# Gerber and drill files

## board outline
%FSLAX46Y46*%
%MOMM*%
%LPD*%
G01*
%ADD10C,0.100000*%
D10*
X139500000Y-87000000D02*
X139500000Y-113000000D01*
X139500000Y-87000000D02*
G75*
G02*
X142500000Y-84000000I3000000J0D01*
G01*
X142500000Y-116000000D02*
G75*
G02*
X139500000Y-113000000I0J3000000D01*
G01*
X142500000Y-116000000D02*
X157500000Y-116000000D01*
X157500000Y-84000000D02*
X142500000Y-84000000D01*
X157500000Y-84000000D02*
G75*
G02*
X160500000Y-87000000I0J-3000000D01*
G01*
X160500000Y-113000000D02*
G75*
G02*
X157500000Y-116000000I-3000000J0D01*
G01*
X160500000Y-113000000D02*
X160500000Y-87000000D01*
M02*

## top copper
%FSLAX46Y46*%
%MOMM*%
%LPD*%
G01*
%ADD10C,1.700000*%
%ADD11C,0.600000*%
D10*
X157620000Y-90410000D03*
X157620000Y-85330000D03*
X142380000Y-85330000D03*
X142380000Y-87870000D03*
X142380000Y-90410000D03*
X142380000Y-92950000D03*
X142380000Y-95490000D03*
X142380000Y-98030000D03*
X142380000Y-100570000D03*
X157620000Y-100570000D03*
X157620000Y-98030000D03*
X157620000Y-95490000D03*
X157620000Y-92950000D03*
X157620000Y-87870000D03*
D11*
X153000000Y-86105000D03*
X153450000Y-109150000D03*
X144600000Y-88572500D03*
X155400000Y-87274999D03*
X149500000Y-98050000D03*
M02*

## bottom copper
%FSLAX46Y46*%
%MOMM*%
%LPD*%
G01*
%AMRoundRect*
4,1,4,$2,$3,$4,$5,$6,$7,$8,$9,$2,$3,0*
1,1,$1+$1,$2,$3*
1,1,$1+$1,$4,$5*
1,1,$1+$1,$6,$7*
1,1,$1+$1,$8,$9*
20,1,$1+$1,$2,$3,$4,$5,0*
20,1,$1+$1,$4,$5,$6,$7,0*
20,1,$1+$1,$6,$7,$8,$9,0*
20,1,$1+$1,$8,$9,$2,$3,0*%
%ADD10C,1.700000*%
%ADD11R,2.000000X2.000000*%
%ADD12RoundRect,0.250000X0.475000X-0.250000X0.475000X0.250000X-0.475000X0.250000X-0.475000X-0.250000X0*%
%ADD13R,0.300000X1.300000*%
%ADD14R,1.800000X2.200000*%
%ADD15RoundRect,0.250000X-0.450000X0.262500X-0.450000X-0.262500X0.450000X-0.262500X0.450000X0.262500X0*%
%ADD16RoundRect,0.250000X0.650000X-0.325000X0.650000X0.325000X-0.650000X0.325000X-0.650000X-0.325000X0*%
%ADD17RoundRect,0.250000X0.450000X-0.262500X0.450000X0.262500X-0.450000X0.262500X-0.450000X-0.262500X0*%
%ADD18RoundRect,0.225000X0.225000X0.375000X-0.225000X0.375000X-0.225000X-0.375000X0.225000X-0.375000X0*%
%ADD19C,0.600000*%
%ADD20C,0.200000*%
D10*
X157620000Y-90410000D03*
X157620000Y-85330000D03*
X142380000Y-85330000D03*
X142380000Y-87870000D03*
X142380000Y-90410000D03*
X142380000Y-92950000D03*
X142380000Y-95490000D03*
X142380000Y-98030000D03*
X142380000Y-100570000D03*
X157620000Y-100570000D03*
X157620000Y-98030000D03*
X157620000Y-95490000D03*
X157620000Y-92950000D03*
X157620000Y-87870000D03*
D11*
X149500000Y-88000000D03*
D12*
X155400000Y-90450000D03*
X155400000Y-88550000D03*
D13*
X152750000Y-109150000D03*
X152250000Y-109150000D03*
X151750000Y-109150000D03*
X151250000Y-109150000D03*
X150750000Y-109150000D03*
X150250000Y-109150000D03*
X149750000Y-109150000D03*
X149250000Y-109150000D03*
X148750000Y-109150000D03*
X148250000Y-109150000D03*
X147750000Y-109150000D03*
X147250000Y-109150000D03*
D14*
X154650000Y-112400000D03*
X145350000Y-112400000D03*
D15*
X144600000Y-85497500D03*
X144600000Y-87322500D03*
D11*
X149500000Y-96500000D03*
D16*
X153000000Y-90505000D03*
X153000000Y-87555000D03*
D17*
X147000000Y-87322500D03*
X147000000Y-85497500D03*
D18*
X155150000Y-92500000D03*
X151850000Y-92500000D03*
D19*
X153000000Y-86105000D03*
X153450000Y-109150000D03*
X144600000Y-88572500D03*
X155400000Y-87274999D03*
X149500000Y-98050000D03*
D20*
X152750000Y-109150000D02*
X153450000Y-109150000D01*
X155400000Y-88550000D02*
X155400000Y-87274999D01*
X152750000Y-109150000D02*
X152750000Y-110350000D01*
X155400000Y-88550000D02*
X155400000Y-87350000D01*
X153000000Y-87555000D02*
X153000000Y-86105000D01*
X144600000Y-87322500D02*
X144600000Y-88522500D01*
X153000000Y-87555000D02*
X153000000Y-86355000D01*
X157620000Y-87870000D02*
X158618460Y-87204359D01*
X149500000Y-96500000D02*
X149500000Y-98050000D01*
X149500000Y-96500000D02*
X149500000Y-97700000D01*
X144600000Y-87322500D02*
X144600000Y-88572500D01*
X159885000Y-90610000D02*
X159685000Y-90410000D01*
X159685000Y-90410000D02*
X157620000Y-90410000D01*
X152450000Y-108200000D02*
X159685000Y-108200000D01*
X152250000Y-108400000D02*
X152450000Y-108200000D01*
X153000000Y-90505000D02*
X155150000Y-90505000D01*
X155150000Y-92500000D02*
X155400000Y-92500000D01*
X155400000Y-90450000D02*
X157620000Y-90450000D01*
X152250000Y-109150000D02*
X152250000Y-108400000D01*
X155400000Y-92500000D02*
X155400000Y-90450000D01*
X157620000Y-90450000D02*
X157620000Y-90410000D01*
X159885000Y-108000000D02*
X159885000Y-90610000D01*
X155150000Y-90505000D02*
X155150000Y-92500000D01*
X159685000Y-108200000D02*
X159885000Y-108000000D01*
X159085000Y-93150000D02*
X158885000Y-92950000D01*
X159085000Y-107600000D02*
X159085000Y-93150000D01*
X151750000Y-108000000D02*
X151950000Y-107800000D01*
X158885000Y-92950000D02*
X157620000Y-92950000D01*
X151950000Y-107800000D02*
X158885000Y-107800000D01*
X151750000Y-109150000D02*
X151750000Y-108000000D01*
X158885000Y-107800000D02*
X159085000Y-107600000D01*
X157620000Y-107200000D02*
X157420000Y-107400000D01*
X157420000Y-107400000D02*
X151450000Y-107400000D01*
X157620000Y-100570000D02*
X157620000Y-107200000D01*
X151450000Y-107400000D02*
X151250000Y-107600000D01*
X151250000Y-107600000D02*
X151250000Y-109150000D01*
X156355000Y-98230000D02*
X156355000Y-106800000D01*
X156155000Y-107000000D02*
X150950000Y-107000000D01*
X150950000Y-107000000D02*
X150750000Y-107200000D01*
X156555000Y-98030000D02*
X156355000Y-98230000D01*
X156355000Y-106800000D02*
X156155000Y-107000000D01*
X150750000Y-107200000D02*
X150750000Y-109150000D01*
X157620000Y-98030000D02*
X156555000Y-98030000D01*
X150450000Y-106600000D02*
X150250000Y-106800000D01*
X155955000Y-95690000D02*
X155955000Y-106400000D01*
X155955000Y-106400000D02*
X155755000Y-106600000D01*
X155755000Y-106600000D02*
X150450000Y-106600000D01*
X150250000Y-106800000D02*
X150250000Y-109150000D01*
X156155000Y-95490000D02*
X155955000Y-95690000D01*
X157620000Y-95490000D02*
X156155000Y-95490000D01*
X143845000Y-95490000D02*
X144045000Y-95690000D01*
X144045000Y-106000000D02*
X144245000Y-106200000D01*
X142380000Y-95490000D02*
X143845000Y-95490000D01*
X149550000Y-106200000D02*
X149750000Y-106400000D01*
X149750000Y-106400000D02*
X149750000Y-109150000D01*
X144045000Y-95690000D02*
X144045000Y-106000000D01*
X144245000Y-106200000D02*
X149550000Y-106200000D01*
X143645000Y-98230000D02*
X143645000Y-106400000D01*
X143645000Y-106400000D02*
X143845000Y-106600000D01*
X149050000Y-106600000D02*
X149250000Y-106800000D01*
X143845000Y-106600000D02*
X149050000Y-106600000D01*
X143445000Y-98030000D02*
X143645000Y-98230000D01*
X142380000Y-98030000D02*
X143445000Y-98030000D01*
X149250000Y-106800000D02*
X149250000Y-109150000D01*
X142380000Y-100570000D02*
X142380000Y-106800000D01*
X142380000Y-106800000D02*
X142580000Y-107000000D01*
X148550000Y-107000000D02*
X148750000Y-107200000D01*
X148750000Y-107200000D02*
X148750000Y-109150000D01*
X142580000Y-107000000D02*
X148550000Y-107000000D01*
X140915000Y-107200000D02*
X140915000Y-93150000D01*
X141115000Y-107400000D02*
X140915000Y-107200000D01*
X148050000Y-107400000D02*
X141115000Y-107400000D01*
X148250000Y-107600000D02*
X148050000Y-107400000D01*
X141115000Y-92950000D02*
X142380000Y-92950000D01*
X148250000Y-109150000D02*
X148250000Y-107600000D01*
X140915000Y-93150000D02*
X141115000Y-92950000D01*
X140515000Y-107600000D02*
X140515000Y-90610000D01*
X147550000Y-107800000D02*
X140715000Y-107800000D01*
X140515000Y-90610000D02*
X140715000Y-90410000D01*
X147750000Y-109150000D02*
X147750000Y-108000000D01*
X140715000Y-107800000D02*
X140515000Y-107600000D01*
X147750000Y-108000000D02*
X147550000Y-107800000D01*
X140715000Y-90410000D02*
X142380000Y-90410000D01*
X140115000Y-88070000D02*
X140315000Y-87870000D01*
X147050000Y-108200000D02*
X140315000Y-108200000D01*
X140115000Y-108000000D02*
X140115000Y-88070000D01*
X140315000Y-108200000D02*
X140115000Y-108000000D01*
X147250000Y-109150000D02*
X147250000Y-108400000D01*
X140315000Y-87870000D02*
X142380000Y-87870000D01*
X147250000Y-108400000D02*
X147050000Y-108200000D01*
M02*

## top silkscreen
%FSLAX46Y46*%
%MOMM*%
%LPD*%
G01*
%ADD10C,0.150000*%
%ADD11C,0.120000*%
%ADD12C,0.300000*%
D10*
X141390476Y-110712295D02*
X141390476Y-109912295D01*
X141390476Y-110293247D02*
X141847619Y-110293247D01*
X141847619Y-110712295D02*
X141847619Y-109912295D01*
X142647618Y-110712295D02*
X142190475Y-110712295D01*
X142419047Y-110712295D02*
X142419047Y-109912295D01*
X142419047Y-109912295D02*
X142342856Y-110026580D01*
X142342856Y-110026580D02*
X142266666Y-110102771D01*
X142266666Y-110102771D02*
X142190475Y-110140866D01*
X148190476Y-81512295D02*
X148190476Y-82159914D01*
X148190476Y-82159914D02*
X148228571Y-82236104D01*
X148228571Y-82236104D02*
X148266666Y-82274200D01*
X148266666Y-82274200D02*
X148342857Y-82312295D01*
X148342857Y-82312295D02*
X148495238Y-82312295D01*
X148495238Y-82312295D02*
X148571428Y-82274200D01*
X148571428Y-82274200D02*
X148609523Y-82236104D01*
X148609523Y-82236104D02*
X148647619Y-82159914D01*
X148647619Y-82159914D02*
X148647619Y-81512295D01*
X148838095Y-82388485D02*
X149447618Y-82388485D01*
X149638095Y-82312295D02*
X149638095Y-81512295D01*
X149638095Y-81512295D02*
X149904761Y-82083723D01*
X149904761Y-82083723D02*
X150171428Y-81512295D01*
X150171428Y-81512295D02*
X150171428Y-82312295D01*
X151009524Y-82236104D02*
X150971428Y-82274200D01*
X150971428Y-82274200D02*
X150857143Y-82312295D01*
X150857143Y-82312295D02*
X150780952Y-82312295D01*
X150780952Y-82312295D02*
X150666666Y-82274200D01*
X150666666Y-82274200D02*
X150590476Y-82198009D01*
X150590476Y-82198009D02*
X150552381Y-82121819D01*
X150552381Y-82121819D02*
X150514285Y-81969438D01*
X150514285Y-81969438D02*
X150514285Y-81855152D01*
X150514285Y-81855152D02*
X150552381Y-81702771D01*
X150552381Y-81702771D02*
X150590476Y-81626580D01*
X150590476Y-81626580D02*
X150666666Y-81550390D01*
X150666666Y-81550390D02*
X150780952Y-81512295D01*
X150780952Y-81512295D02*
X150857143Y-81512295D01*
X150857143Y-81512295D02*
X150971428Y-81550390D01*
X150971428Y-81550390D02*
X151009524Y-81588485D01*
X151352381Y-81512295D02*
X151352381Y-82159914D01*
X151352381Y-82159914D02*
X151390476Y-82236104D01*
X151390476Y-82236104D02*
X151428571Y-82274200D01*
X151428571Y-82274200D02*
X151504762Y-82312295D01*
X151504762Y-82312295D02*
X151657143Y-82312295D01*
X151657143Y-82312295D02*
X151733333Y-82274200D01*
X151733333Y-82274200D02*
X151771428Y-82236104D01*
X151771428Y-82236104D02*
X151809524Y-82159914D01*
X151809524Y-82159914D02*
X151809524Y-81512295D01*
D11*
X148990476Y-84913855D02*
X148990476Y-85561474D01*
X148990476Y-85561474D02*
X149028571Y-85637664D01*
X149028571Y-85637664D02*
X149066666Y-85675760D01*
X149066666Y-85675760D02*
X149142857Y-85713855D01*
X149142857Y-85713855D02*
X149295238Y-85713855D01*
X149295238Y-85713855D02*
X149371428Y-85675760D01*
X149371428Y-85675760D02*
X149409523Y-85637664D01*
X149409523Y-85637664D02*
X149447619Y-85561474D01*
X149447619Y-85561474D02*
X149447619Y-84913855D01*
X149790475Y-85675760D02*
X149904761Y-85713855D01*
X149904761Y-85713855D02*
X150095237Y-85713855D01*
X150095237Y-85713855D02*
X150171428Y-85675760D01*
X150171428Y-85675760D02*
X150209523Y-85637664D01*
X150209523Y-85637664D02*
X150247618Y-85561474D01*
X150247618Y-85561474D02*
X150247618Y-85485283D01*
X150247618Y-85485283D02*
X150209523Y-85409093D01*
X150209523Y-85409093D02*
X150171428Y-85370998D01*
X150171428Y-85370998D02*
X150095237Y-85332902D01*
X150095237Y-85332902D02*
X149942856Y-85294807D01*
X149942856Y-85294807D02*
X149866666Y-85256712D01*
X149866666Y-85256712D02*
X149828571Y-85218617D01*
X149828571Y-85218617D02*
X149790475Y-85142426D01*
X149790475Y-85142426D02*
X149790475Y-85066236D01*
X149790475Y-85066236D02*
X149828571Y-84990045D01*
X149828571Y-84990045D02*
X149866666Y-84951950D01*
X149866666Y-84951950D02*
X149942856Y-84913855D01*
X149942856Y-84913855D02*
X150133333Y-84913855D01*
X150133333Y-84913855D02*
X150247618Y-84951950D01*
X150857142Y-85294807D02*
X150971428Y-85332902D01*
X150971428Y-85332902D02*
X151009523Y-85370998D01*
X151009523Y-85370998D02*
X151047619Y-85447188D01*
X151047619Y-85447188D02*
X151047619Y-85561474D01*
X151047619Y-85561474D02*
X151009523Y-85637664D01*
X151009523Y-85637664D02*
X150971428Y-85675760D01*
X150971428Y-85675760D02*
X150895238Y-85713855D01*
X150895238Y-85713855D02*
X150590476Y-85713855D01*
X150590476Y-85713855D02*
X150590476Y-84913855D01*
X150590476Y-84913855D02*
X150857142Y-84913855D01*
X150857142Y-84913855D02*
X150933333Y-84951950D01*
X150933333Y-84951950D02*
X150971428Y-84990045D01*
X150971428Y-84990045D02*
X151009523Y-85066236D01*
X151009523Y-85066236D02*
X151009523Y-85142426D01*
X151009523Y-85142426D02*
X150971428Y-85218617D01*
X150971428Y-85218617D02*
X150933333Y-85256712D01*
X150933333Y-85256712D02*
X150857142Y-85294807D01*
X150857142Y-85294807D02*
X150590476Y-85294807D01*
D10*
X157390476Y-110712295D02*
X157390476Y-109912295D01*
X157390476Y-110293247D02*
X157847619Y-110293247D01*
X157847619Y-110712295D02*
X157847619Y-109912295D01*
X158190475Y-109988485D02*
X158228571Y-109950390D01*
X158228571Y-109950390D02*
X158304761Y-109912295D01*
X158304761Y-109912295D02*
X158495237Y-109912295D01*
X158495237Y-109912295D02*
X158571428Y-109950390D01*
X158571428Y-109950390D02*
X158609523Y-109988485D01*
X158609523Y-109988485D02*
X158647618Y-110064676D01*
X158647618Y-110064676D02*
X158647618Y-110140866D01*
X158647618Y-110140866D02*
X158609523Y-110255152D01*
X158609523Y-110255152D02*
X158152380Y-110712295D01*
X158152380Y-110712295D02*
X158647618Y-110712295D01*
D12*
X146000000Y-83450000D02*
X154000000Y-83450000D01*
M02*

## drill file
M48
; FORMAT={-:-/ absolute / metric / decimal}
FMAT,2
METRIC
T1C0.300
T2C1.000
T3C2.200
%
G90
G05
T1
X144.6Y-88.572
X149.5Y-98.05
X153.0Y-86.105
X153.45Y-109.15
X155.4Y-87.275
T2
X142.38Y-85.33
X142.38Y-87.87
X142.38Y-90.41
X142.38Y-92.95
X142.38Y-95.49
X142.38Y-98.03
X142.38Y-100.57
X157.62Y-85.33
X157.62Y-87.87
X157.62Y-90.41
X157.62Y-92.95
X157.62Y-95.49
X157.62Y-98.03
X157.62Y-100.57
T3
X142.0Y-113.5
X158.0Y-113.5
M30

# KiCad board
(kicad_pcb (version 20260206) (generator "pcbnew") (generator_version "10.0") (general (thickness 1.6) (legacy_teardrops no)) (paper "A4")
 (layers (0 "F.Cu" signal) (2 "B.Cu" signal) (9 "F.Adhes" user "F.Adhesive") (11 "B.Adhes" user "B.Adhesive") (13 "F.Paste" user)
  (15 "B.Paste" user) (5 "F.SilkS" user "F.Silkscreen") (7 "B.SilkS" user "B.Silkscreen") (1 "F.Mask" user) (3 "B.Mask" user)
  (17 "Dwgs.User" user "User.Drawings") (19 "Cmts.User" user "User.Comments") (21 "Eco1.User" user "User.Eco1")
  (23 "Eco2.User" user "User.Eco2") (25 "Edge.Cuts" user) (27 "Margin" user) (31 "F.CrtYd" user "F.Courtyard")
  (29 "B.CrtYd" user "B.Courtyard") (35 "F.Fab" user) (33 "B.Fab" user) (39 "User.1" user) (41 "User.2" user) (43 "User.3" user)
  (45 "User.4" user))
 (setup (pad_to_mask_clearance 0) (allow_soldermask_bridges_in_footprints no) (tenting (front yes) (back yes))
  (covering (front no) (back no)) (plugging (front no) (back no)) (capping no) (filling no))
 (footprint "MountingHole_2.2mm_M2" (layer "F.Cu") (at 142 113.5)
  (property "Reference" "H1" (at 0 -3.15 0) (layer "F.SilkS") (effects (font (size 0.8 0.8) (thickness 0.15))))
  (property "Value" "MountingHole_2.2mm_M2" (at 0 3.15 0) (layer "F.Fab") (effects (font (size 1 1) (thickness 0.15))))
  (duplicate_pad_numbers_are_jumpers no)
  (pad "" np_thru_hole circle (at 0 0) (size 2.2 2.2) (drill 2.2) (layers "*.Cu" "*.Mask")))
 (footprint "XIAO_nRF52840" (layer "F.Cu") (at 150 92.95)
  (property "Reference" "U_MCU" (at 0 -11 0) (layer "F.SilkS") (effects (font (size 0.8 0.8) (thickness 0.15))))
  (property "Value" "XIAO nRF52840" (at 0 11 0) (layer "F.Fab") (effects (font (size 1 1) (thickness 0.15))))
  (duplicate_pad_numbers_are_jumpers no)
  (fp_line (start -4 -9.5) (end 4 -9.5) (stroke (width 0.3) (type solid)) (layer "F.SilkS"))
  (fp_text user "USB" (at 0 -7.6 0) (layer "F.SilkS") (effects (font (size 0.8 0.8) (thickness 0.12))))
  (pad "3V3" thru_hole circle (at 7.62 -2.54) (size 1.7 1.7) (drill 1) (layers "*.Cu" "*.Mask") (remove_unused_layers no) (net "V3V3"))
  (pad "5V" thru_hole circle (at 7.62 -7.62) (size 1.7 1.7) (drill 1) (layers "*.Cu" "*.Mask") (remove_unused_layers no))
  (pad "D0" thru_hole circle (at -7.62 -7.62) (size 1.7 1.7) (drill 1) (layers "*.Cu" "*.Mask") (remove_unused_layers no)
   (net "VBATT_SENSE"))
  (pad "D1" thru_hole circle (at -7.62 -5.08) (size 1.7 1.7) (drill 1) (layers "*.Cu" "*.Mask") (remove_unused_layers no) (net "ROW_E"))
  (pad "D2" thru_hole circle (at -7.62 -2.54) (size 1.7 1.7) (drill 1) (layers "*.Cu" "*.Mask") (remove_unused_layers no) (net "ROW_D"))
  (pad "D3" thru_hole circle (at -7.62 0) (size 1.7 1.7) (drill 1) (layers "*.Cu" "*.Mask") (remove_unused_layers no) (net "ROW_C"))
  (pad "D4" thru_hole circle (at -7.62 2.54) (size 1.7 1.7) (drill 1) (layers "*.Cu" "*.Mask") (remove_unused_layers no) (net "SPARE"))
  (pad "D5" thru_hole circle (at -7.62 5.08) (size 1.7 1.7) (drill 1) (layers "*.Cu" "*.Mask") (remove_unused_layers no) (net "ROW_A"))
  (pad "D6" thru_hole circle (at -7.62 7.62) (size 1.7 1.7) (drill 1) (layers "*.Cu" "*.Mask") (remove_unused_layers no) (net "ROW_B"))
  (pad "D7" thru_hole circle (at 7.62 7.62) (size 1.7 1.7) (drill 1) (layers "*.Cu" "*.Mask") (remove_unused_layers no) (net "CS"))
  (pad "D8" thru_hole circle (at 7.62 5.08) (size 1.7 1.7) (drill 1) (layers "*.Cu" "*.Mask") (remove_unused_layers no) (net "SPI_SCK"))
  (pad "D9" thru_hole circle (at 7.62 2.54) (size 1.7 1.7) (drill 1) (layers "*.Cu" "*.Mask") (remove_unused_layers no) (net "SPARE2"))
  (pad "D10" thru_hole circle (at 7.62 0) (size 1.7 1.7) (drill 1) (layers "*.Cu" "*.Mask") (remove_unused_layers no) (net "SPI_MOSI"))
  (pad "GND" thru_hole circle (at 7.62 -5.08) (size 1.7 1.7) (drill 1) (layers "*.Cu" "*.Mask") (remove_unused_layers no) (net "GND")))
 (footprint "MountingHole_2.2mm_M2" (layer "F.Cu") (at 158 113.5)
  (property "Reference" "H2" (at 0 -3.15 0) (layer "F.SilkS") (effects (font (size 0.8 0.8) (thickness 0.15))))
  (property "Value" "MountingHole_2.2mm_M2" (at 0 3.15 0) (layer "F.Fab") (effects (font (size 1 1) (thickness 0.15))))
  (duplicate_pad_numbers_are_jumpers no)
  (pad "" np_thru_hole circle (at 0 0) (size 2.2 2.2) (drill 2.2) (layers "*.Cu" "*.Mask")))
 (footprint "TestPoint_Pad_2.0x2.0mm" (layer "B.Cu") (at 149.5 88 180)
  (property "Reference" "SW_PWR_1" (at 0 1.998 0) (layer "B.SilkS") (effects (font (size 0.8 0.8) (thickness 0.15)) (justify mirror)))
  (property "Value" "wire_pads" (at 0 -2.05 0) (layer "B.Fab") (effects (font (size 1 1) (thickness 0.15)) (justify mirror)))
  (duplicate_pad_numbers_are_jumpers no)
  (pad "1" smd rect (at 0 0 180) (size 2 2) (layers "B.Cu" "B.Mask") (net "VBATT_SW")))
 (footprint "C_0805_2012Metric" (layer "B.Cu") (at 155.4 89.5 90)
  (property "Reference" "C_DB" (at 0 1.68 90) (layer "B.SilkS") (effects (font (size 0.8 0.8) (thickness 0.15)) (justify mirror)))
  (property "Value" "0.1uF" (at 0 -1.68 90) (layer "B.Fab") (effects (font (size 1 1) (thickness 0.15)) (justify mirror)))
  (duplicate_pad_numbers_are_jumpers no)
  (pad "1" smd roundrect (at -0.95 0 90) (size 1 1.45) (layers "B.Cu" "B.Mask" "B.Paste") (roundrect_rratio 0.25) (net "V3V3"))
  (pad "2" smd roundrect (at 0.95 0 90) (size 1 1.45) (layers "B.Cu" "B.Mask" "B.Paste") (roundrect_rratio 0.25) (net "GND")))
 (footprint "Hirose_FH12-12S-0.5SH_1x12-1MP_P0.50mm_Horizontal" (layer "B.Cu") (at 150 111 180)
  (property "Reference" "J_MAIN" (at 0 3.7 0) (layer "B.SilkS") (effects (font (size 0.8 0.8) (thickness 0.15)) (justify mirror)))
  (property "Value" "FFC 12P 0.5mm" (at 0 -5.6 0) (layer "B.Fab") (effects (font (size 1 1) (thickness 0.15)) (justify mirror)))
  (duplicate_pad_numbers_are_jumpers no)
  (pad "1" smd rect (at -2.75 1.85 180) (size 0.3 1.3) (layers "B.Cu" "B.Mask" "B.Paste") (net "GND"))
  (pad "2" smd rect (at -2.25 1.85 180) (size 0.3 1.3) (layers "B.Cu" "B.Mask" "B.Paste") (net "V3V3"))
  (pad "3" smd rect (at -1.75 1.85 180) (size 0.3 1.3) (layers "B.Cu" "B.Mask" "B.Paste") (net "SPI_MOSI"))
  (pad "4" smd rect (at -1.25 1.85 180) (size 0.3 1.3) (layers "B.Cu" "B.Mask" "B.Paste") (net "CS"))
  (pad "5" smd rect (at -0.75 1.85 180) (size 0.3 1.3) (layers "B.Cu" "B.Mask" "B.Paste") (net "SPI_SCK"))
  (pad "6" smd rect (at -0.25 1.85 180) (size 0.3 1.3) (layers "B.Cu" "B.Mask" "B.Paste") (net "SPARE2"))
  (pad "7" smd rect (at 0.25 1.85 180) (size 0.3 1.3) (layers "B.Cu" "B.Mask" "B.Paste") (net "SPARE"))
  (pad "8" smd rect (at 0.75 1.85 180) (size 0.3 1.3) (layers "B.Cu" "B.Mask" "B.Paste") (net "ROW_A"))
  (pad "9" smd rect (at 1.25 1.85 180) (size 0.3 1.3) (layers "B.Cu" "B.Mask" "B.Paste") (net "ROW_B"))
  (pad "10" smd rect (at 1.75 1.85 180) (size 0.3 1.3) (layers "B.Cu" "B.Mask" "B.Paste") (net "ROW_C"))
  (pad "11" smd rect (at 2.25 1.85 180) (size 0.3 1.3) (layers "B.Cu" "B.Mask" "B.Paste") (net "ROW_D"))
  (pad "12" smd rect (at 2.75 1.85 180) (size 0.3 1.3) (layers "B.Cu" "B.Mask" "B.Paste") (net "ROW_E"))
  (pad "MP" smd rect (at -4.65 -1.4 180) (size 1.8 2.2) (layers "B.Cu" "B.Mask" "B.Paste"))
  (pad "MP" smd rect (at 4.65 -1.4 180) (size 1.8 2.2) (layers "B.Cu" "B.Mask" "B.Paste")))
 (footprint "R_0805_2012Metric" (layer "B.Cu") (at 144.6 86.41 -90)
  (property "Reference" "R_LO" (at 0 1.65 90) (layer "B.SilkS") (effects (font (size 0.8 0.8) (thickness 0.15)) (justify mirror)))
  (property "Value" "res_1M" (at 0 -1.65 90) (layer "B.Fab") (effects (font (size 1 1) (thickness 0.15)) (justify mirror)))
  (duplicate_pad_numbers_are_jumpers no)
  (pad "1" smd roundrect (at -0.9125 0 270) (size 1.025 1.4) (layers "B.Cu" "B.Mask" "B.Paste") (roundrect_rratio 0.243902)
   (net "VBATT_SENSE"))
  (pad "2" smd roundrect (at 0.9125 0 270) (size 1.025 1.4) (layers "B.Cu" "B.Mask" "B.Paste") (roundrect_rratio 0.243902) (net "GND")))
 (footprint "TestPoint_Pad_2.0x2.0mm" (layer "B.Cu") (at 149.5 96.5 180)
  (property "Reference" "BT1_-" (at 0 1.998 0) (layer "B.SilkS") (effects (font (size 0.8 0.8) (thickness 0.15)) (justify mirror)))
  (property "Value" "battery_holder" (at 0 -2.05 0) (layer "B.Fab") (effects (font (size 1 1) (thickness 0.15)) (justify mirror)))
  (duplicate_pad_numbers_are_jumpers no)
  (pad "1" smd rect (at 0 0 180) (size 2 2) (layers "B.Cu" "B.Mask") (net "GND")))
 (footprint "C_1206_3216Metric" (layer "B.Cu") (at 153 89.03 90)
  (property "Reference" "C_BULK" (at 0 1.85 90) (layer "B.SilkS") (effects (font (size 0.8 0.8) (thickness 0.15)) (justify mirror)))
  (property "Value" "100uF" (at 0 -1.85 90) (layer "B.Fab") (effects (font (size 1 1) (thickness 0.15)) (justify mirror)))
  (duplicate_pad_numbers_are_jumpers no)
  (pad "1" smd roundrect (at -1.475 0 90) (size 1.15 1.8) (layers "B.Cu" "B.Mask" "B.Paste") (roundrect_rratio 0.217391) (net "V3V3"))
  (pad "2" smd roundrect (at 1.475 0 90) (size 1.15 1.8) (layers "B.Cu" "B.Mask" "B.Paste") (roundrect_rratio 0.217391) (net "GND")))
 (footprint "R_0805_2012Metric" (layer "B.Cu") (at 147 86.41 90)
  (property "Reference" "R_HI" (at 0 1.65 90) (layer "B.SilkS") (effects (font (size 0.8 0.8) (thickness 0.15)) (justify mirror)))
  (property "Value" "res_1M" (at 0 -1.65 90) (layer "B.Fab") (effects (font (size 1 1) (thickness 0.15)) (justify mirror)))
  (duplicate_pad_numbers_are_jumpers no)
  (pad "1" smd roundrect (at -0.9125 0 90) (size 1.025 1.4) (layers "B.Cu" "B.Mask" "B.Paste") (roundrect_rratio 0.243902) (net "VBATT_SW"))
  (pad "2" smd roundrect (at 0.9125 0 90) (size 1.025 1.4) (layers "B.Cu" "B.Mask" "B.Paste") (roundrect_rratio 0.243902)
   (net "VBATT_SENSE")))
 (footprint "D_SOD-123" (layer "B.Cu") (at 153.5 92.5 180)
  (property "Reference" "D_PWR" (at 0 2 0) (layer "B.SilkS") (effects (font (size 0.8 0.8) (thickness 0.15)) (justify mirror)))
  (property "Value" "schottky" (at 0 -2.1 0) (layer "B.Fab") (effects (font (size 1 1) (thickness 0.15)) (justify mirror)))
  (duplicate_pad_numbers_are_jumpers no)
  (pad "1" smd roundrect (at -1.65 0 180) (size 0.9 1.2) (layers "B.Cu" "B.Mask" "B.Paste") (roundrect_rratio 0.25) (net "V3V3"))
  (pad "2" smd roundrect (at 1.65 0 180) (size 0.9 1.2) (layers "B.Cu" "B.Mask" "B.Paste") (roundrect_rratio 0.25) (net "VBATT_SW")))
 (gr_line (start 139.5 87) (end 139.5 113) (stroke (width 0.1) (type default)) (layer "Edge.Cuts"))
 (gr_arc (start 139.5 87) (mid 140.37868 84.87868) (end 142.5 84) (stroke (width 0.1) (type default)) (layer "Edge.Cuts"))
 (gr_arc (start 142.5 116) (mid 140.37868 115.12132) (end 139.5 113) (stroke (width 0.1) (type default)) (layer "Edge.Cuts"))
 (gr_line (start 142.5 116) (end 157.5 116) (stroke (width 0.1) (type default)) (layer "Edge.Cuts"))
 (gr_line (start 157.5 84) (end 142.5 84) (stroke (width 0.1) (type default)) (layer "Edge.Cuts"))
 (gr_arc (start 157.5 84) (mid 159.62132 84.87868) (end 160.5 87) (stroke (width 0.1) (type default)) (layer "Edge.Cuts"))
 (gr_arc (start 160.5 113) (mid 159.62132 115.12132) (end 157.5 116) (stroke (width 0.1) (type default)) (layer "Edge.Cuts"))
 (gr_line (start 160.5 113) (end 160.5 87) (stroke (width 0.1) (type default)) (layer "Edge.Cuts"))
 (via (at 153 86.105) (size 0.6) (drill 0.3) (layers "F.Cu" "B.Cu") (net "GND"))
 (via (at 153.45 109.15) (size 0.6) (drill 0.3) (layers "F.Cu" "B.Cu") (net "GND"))
 (via (at 144.6 88.5725) (size 0.6) (drill 0.3) (layers "F.Cu" "B.Cu") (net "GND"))
 (via (at 155.4 87.274999) (size 0.6) (drill 0.3) (layers "F.Cu" "B.Cu") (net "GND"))
 (via (at 149.5 98.05) (size 0.6) (drill 0.3) (layers "F.Cu" "B.Cu") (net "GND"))
 (segment (start 152.75 109.15) (end 153.45 109.15) (width 0.2) (layer "B.Cu") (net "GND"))
 (segment (start 155.4 88.55) (end 155.4 87.274999) (width 0.2) (layer "B.Cu") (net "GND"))
 (segment (start 152.75 109.15) (end 152.75 110.35) (width 0.2) (layer "B.Cu") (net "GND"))
 (segment (start 155.4 88.55) (end 155.4 87.35) (width 0.2) (layer "B.Cu") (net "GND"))
 (segment (start 153 87.555) (end 153 86.105) (width 0.2) (layer "B.Cu") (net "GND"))
 (segment (start 144.6 87.3225) (end 144.6 88.5225) (width 0.2) (layer "B.Cu") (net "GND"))
 (segment (start 153 87.555) (end 153 86.355) (width 0.2) (layer "B.Cu") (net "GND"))
 (segment (start 157.62 87.87) (end 158.61846 87.204359) (width 0.2) (layer "B.Cu") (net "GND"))
 (segment (start 149.5 96.5) (end 149.5 98.05) (width 0.2) (layer "B.Cu") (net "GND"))
 (segment (start 149.5 96.5) (end 149.5 97.7) (width 0.2) (layer "B.Cu") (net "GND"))
 (segment (start 144.6 87.3225) (end 144.6 88.5725) (width 0.2) (layer "B.Cu") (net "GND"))
 (segment (start 159.885 90.61) (end 159.685 90.41) (width 0.2) (layer "B.Cu") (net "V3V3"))
 (segment (start 159.685 90.41) (end 157.62 90.41) (width 0.2) (layer "B.Cu") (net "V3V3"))
 (segment (start 152.45 108.2) (end 159.685 108.2) (width 0.2) (layer "B.Cu") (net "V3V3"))
 (segment (start 152.25 108.4) (end 152.45 108.2) (width 0.2) (layer "B.Cu") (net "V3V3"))
 (segment (start 153 90.505) (end 155.15 90.505) (width 0.2) (layer "B.Cu") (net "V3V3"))
 (segment (start 155.15 92.5) (end 155.4 92.5) (width 0.2) (layer "B.Cu") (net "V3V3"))
 (segment (start 155.4 90.45) (end 157.62 90.45) (width 0.2) (layer "B.Cu") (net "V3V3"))
 (segment (start 152.25 109.15) (end 152.25 108.4) (width 0.2) (layer "B.Cu") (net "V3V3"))
 (segment (start 155.4 92.5) (end 155.4 90.45) (width 0.2) (layer "B.Cu") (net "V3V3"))
 (segment (start 157.62 90.45) (end 157.62 90.41) (width 0.2) (layer "B.Cu") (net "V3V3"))
 (segment (start 159.885 108) (end 159.885 90.61) (width 0.2) (layer "B.Cu") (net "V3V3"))
 (segment (start 155.15 90.505) (end 155.15 92.5) (width 0.2) (layer "B.Cu") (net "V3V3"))
 (segment (start 159.685 108.2) (end 159.885 108) (width 0.2) (layer "B.Cu") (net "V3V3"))
 (segment (start 159.085 93.15) (end 158.885 92.95) (width 0.2) (layer "B.Cu") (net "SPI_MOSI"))
 (segment (start 159.085 107.6) (end 159.085 93.15) (width 0.2) (layer "B.Cu") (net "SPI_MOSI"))
 (segment (start 151.75 108) (end 151.95 107.8) (width 0.2) (layer "B.Cu") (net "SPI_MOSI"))
 (segment (start 158.885 92.95) (end 157.62 92.95) (width 0.2) (layer "B.Cu") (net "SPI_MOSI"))
 (segment (start 151.95 107.8) (end 158.885 107.8) (width 0.2) (layer "B.Cu") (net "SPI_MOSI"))
 (segment (start 151.75 109.15) (end 151.75 108) (width 0.2) (layer "B.Cu") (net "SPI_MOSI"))
 (segment (start 158.885 107.8) (end 159.085 107.6) (width 0.2) (layer "B.Cu") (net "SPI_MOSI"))
 (segment (start 157.62 107.2) (end 157.42 107.4) (width 0.2) (layer "B.Cu") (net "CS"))
 (segment (start 157.42 107.4) (end 151.45 107.4) (width 0.2) (layer "B.Cu") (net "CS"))
 (segment (start 157.62 100.57) (end 157.62 107.2) (width 0.2) (layer "B.Cu") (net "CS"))
 (segment (start 151.45 107.4) (end 151.25 107.6) (width 0.2) (layer "B.Cu") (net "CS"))
 (segment (start 151.25 107.6) (end 151.25 109.15) (width 0.2) (layer "B.Cu") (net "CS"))
 (segment (start 156.355 98.23) (end 156.355 106.8) (width 0.2) (layer "B.Cu") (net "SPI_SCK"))
 (segment (start 156.155 107) (end 150.95 107) (width 0.2) (layer "B.Cu") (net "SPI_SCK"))
 (segment (start 150.95 107) (end 150.75 107.2) (width 0.2) (layer "B.Cu") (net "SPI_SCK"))
 (segment (start 156.555 98.03) (end 156.355 98.23) (width 0.2) (layer "B.Cu") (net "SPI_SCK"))
 (segment (start 156.355 106.8) (end 156.155 107) (width 0.2) (layer "B.Cu") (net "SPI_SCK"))
 (segment (start 150.75 107.2) (end 150.75 109.15) (width 0.2) (layer "B.Cu") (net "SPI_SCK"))
 (segment (start 157.62 98.03) (end 156.555 98.03) (width 0.2) (layer "B.Cu") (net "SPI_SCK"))
 (segment (start 150.45 106.6) (end 150.25 106.8) (width 0.2) (layer "B.Cu") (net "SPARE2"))
 (segment (start 155.955 95.69) (end 155.955 106.4) (width 0.2) (layer "B.Cu") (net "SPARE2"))
 (segment (start 155.955 106.4) (end 155.755 106.6) (width 0.2) (layer "B.Cu") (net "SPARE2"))
 (segment (start 155.755 106.6) (end 150.45 106.6) (width 0.2) (layer "B.Cu") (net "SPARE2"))
 (segment (start 150.25 106.8) (end 150.25 109.15) (width 0.2) (layer "B.Cu") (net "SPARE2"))
 (segment (start 156.155 95.49) (end 155.955 95.69) (width 0.2) (layer "B.Cu") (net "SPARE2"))
 (segment (start 157.62 95.49) (end 156.155 95.49) (width 0.2) (layer "B.Cu") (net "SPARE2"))
 (segment (start 143.845 95.49) (end 144.045 95.69) (width 0.2) (layer "B.Cu") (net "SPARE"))
 (segment (start 144.045 106) (end 144.245 106.2) (width 0.2) (layer "B.Cu") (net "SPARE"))
 (segment (start 142.38 95.49) (end 143.845 95.49) (width 0.2) (layer "B.Cu") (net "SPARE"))
 (segment (start 149.55 106.2) (end 149.75 106.4) (width 0.2) (layer "B.Cu") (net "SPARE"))
 (segment (start 149.75 106.4) (end 149.75 109.15) (width 0.2) (layer "B.Cu") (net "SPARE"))
 (segment (start 144.045 95.69) (end 144.045 106) (width 0.2) (layer "B.Cu") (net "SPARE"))
 (segment (start 144.245 106.2) (end 149.55 106.2) (width 0.2) (layer "B.Cu") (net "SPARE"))
 (segment (start 143.645 98.23) (end 143.645 106.4) (width 0.2) (layer "B.Cu") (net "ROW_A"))
 (segment (start 143.645 106.4) (end 143.845 106.6) (width 0.2) (layer "B.Cu") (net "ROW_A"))
 (segment (start 149.05 106.6) (end 149.25 106.8) (width 0.2) (layer "B.Cu") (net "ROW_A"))
 (segment (start 143.845 106.6) (end 149.05 106.6) (width 0.2) (layer "B.Cu") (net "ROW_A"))
 (segment (start 143.445 98.03) (end 143.645 98.23) (width 0.2) (layer "B.Cu") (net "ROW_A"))
 (segment (start 142.38 98.03) (end 143.445 98.03) (width 0.2) (layer "B.Cu") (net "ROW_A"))
 (segment (start 149.25 106.8) (end 149.25 109.15) (width 0.2) (layer "B.Cu") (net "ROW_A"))
 (segment (start 142.38 100.57) (end 142.38 106.8) (width 0.2) (layer "B.Cu") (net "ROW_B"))
 (segment (start 142.38 106.8) (end 142.58 107) (width 0.2) (layer "B.Cu") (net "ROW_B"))
 (segment (start 148.55 107) (end 148.75 107.2) (width 0.2) (layer "B.Cu") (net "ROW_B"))
 (segment (start 148.75 107.2) (end 148.75 109.15) (width 0.2) (layer "B.Cu") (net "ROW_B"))
 (segment (start 142.58 107) (end 148.55 107) (width 0.2) (layer "B.Cu") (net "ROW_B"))
 (segment (start 140.915 107.2) (end 140.915 93.15) (width 0.2) (layer "B.Cu") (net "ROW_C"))
 (segment (start 141.115 107.4) (end 140.915 107.2) (width 0.2) (layer "B.Cu") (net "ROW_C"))
 (segment (start 148.05 107.4) (end 141.115 107.4) (width 0.2) (layer "B.Cu") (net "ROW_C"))
 (segment (start 148.25 107.6) (end 148.05 107.4) (width 0.2) (layer "B.Cu") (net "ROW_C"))
 (segment (start 141.115 92.95) (end 142.38 92.95) (width 0.2) (layer "B.Cu") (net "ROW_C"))
 (segment (start 148.25 109.15) (end 148.25 107.6) (width 0.2) (layer "B.Cu") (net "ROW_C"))
 (segment (start 140.915 93.15) (end 141.115 92.95) (width 0.2) (layer "B.Cu") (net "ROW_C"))
 (segment (start 140.515 107.6) (end 140.515 90.61) (width 0.2) (layer "B.Cu") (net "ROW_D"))
 (segment (start 147.55 107.8) (end 140.715 107.8) (width 0.2) (layer "B.Cu") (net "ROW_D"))
 (segment (start 140.515 90.61) (end 140.715 90.41) (width 0.2) (layer "B.Cu") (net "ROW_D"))
 (segment (start 147.75 109.15) (end 147.75 108) (width 0.2) (layer "B.Cu") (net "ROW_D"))
 (segment (start 140.715 107.8) (end 140.515 107.6) (width 0.2) (layer "B.Cu") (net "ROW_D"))
 (segment (start 147.75 108) (end 147.55 107.8) (width 0.2) (layer "B.Cu") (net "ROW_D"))
 (segment (start 140.715 90.41) (end 142.38 90.41) (width 0.2) (layer "B.Cu") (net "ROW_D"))
 (segment (start 140.115 88.07) (end 140.315 87.87) (width 0.2) (layer "B.Cu") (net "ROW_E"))
 (segment (start 147.05 108.2) (end 140.315 108.2) (width 0.2) (layer "B.Cu") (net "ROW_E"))
 (segment (start 140.115 108) (end 140.115 88.07) (width 0.2) (layer "B.Cu") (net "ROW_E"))
 (segment (start 140.315 108.2) (end 140.115 108) (width 0.2) (layer "B.Cu") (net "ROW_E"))
 (segment (start 147.25 109.15) (end 147.25 108.4) (width 0.2) (layer "B.Cu") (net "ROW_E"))
 (segment (start 140.315 87.87) (end 142.38 87.87) (width 0.2) (layer "B.Cu") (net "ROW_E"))
 (segment (start 147.25 108.4) (end 147.05 108.2) (width 0.2) (layer "B.Cu") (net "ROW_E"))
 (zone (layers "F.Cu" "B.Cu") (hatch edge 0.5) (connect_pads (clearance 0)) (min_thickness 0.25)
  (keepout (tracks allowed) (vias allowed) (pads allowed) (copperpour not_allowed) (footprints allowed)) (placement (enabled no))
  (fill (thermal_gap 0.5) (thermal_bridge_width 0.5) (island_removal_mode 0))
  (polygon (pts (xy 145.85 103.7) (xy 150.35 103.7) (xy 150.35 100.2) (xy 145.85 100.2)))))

